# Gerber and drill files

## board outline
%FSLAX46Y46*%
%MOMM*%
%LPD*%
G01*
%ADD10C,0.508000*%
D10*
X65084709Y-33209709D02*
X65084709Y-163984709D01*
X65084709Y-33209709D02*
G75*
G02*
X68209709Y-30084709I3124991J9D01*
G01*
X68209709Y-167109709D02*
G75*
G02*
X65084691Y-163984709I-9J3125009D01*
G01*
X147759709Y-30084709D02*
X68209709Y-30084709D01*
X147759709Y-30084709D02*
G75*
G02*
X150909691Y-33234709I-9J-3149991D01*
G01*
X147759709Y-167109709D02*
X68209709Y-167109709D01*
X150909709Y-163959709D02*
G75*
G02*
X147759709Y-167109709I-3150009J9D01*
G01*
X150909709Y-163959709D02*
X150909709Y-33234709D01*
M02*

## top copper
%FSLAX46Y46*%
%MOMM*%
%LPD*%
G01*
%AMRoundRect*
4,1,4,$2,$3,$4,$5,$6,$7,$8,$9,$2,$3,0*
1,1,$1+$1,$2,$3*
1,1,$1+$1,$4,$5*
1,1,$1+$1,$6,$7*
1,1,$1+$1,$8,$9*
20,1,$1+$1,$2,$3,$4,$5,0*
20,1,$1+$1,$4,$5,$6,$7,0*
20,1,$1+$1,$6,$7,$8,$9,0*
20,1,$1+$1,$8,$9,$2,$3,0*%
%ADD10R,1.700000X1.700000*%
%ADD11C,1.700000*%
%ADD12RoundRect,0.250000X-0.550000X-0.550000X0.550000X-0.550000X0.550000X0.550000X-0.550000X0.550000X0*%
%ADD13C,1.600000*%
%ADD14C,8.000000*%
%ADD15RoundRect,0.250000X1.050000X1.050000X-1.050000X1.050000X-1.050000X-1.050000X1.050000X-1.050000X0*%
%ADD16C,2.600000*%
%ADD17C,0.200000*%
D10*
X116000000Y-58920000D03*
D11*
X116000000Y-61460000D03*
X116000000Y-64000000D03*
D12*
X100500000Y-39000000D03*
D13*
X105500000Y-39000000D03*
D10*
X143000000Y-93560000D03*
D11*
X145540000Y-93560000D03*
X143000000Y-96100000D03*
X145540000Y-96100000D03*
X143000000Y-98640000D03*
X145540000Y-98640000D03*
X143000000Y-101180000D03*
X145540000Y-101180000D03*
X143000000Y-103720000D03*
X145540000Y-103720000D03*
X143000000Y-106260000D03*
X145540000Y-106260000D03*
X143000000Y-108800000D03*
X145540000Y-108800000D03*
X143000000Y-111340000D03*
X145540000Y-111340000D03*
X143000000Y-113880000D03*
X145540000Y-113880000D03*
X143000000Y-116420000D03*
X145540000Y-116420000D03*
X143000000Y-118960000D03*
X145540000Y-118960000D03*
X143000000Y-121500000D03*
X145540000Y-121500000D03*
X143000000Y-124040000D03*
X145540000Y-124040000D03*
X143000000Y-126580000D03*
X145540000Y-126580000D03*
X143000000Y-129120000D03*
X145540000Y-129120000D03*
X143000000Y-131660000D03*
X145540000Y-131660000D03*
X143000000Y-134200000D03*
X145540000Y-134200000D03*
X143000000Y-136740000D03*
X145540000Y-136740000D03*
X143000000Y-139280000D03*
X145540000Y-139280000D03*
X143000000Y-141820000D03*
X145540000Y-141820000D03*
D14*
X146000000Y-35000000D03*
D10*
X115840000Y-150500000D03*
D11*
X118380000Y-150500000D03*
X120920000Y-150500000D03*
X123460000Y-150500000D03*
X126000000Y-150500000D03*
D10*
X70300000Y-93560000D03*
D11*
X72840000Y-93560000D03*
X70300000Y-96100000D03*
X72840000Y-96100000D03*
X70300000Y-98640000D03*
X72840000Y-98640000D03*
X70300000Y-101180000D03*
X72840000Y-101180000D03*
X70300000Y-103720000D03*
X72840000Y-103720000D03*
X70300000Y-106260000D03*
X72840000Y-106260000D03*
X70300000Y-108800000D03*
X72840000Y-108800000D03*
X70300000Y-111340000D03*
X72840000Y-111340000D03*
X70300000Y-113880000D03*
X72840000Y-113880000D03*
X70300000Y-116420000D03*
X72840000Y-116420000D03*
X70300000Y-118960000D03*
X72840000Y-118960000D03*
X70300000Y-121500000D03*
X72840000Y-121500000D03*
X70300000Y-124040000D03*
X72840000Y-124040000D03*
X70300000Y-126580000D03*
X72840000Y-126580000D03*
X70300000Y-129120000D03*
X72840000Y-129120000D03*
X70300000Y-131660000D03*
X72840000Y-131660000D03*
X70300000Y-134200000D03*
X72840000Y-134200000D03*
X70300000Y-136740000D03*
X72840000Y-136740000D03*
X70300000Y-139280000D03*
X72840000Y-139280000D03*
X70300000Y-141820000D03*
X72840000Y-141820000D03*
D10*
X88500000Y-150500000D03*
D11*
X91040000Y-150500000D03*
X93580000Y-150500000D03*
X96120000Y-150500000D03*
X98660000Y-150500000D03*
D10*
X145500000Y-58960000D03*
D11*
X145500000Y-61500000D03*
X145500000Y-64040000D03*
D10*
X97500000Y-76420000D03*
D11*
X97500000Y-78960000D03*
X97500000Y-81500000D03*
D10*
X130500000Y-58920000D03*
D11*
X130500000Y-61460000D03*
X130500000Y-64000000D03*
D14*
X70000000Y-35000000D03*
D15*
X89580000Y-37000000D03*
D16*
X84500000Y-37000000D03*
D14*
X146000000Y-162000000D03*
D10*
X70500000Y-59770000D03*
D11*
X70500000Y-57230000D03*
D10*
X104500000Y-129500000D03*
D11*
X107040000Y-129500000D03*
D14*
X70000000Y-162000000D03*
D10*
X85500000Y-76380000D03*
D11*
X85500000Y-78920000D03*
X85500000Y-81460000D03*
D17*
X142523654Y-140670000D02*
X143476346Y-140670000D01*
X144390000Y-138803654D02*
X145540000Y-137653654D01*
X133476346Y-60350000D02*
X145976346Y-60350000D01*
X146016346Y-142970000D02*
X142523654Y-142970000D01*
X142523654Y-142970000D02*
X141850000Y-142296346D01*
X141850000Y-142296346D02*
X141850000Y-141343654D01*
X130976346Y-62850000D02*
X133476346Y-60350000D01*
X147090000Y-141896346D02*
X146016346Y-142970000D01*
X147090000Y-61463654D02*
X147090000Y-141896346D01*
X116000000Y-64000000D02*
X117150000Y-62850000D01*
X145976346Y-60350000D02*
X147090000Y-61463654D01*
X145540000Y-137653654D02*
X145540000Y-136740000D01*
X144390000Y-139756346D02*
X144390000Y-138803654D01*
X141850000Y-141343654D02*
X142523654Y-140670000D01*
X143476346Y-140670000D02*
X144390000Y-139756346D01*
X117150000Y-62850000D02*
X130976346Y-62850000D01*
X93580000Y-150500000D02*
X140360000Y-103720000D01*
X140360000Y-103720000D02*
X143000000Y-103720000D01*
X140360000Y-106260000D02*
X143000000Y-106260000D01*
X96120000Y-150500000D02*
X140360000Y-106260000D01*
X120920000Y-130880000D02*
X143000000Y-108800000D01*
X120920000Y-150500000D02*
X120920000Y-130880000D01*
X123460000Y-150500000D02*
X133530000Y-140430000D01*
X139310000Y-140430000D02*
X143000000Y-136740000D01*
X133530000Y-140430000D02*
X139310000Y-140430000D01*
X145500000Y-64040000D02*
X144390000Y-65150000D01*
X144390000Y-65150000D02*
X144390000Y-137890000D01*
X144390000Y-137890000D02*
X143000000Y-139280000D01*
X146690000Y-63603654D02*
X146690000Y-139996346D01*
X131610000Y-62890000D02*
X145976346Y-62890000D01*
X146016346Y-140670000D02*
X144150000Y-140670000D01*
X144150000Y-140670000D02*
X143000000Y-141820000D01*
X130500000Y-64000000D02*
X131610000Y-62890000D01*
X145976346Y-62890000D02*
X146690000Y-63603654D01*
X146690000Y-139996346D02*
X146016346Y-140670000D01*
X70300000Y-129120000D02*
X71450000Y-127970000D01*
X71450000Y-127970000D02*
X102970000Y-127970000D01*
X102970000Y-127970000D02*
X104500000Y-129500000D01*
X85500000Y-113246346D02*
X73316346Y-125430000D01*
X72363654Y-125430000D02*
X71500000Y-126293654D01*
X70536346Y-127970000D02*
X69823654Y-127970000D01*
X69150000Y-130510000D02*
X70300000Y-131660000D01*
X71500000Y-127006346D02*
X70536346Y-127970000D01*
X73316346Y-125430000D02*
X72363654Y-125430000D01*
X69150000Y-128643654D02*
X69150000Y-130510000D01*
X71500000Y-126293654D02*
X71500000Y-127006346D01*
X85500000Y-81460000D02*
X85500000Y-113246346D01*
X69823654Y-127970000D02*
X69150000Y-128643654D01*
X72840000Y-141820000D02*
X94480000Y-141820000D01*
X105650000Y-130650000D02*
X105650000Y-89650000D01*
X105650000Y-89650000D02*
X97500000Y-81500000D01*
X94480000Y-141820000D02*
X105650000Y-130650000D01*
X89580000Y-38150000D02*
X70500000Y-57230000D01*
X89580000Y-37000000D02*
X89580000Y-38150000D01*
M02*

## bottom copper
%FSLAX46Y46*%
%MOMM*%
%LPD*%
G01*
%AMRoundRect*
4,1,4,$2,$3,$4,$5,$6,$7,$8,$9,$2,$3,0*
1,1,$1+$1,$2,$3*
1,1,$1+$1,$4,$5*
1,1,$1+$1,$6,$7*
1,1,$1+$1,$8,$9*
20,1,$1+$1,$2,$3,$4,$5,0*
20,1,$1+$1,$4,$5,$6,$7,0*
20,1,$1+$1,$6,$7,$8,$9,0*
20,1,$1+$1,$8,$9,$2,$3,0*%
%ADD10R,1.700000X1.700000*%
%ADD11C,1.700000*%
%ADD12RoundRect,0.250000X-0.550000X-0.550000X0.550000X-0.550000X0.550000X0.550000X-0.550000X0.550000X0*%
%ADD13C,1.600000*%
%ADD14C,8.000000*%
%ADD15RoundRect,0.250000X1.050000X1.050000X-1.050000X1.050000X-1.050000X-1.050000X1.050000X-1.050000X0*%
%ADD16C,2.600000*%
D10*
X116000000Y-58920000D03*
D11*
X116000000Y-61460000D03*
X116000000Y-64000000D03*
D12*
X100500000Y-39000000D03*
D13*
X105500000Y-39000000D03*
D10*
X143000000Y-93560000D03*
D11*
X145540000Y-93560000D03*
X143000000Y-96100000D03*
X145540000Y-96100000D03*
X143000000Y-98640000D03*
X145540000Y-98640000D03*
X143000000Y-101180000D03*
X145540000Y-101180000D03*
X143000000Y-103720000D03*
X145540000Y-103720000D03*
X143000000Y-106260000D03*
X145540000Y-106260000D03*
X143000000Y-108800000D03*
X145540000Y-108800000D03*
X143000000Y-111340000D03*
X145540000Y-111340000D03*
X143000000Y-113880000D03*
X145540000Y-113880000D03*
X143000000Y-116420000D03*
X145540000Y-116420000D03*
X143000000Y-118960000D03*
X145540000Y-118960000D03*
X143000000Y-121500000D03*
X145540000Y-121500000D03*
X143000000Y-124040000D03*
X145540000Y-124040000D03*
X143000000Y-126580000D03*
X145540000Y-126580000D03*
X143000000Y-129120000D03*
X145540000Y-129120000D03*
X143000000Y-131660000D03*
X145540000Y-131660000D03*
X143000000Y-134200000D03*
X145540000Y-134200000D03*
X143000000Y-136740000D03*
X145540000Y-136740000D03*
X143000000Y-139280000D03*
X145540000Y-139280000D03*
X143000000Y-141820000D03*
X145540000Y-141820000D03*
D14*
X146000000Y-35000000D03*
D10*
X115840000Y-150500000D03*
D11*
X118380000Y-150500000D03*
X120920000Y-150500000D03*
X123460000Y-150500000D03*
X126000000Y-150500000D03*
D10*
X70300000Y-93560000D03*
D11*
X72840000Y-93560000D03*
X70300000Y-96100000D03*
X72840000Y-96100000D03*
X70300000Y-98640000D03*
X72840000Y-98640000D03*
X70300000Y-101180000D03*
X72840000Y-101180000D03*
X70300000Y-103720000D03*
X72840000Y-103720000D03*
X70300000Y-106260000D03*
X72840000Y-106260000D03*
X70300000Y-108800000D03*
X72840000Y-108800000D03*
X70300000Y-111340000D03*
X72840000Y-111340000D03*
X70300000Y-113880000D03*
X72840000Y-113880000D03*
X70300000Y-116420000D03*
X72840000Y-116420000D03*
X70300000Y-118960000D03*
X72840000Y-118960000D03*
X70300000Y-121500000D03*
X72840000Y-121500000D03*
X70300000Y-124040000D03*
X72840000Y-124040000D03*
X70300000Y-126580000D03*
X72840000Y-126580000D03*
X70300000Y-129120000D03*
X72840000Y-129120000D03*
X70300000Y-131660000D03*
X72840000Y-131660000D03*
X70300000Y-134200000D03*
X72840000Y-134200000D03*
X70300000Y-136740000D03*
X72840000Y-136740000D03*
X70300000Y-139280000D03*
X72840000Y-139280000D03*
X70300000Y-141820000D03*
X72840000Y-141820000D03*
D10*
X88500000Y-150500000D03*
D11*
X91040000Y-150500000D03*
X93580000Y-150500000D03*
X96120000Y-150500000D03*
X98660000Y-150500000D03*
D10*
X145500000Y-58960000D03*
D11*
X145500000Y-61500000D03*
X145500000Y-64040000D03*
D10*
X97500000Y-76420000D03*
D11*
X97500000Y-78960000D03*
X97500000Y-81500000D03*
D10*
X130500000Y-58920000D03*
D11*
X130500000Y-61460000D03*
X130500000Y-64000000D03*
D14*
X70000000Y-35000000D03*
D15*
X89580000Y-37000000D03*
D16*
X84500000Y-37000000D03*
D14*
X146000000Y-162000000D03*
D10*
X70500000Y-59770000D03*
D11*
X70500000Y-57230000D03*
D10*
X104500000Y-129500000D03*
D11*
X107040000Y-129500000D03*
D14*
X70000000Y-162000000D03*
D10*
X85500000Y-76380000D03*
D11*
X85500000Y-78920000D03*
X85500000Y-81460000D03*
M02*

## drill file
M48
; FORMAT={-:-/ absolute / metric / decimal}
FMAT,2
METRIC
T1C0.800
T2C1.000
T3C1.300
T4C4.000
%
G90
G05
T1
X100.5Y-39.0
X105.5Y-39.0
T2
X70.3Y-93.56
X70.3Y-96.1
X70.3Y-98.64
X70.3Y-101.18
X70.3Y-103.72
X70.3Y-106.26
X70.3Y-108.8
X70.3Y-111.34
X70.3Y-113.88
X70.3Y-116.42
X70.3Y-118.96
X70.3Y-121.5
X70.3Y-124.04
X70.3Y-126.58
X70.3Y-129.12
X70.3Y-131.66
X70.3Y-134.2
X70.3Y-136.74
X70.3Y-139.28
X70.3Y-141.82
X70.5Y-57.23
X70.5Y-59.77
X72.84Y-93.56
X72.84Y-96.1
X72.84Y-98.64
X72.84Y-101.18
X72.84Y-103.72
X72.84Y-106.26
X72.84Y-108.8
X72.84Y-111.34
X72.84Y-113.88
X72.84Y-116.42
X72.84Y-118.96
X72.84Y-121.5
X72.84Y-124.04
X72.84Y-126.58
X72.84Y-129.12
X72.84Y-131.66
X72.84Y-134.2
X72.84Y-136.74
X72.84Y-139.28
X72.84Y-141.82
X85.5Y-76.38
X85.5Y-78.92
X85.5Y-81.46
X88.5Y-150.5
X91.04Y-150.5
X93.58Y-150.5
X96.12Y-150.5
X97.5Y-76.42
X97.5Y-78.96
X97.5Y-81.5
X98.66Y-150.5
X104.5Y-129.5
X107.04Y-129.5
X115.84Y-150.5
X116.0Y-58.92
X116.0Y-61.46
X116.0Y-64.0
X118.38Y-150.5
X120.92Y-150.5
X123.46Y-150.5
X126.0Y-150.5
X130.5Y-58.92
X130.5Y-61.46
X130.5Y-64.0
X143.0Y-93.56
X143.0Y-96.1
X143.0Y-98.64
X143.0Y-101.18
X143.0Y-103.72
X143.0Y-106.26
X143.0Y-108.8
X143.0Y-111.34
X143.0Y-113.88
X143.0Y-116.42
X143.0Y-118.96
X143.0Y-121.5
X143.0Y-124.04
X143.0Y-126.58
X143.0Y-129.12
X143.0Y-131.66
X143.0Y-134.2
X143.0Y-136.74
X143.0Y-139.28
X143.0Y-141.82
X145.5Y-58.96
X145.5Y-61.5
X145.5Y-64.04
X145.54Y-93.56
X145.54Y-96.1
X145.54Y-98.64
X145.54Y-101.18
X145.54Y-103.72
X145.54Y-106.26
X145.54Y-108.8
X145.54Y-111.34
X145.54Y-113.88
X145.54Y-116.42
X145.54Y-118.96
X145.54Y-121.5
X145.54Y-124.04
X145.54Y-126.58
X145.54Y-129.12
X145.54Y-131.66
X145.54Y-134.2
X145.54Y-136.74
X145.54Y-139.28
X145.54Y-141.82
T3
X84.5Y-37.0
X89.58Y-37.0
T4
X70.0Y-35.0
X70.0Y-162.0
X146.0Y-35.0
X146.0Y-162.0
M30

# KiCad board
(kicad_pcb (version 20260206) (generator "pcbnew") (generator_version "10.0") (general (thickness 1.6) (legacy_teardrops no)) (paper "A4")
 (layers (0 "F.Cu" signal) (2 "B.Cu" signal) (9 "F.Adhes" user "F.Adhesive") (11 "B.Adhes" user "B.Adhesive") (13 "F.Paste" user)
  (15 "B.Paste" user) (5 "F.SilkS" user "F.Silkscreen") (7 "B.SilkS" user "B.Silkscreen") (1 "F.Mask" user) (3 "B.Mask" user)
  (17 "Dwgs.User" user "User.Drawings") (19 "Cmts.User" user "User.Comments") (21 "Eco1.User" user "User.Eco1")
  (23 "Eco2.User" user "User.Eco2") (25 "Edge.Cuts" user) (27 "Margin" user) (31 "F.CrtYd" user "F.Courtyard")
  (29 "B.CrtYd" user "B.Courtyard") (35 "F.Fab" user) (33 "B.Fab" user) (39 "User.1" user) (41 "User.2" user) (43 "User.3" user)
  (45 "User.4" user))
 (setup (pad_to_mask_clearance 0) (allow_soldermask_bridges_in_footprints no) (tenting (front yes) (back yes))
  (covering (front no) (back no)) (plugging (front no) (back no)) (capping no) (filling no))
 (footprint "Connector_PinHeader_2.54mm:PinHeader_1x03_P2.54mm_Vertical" (layer "F.Cu") (at 116 58.92)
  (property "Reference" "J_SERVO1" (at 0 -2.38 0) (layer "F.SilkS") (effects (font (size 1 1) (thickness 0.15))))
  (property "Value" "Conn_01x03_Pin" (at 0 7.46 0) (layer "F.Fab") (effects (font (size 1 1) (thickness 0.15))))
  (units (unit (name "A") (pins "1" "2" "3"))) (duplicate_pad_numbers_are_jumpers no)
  (pad "1" thru_hole rect (at 0 0) (size 1.7 1.7) (drill 1) (layers "*.Cu" "*.Mask") (remove_unused_layers no) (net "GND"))
  (pad "2" thru_hole circle (at 0 2.54) (size 1.7 1.7) (drill 1) (layers "*.Cu" "*.Mask") (remove_unused_layers no) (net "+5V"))
  (pad "3" thru_hole circle (at 0 5.08) (size 1.7 1.7) (drill 1) (layers "*.Cu" "*.Mask") (remove_unused_layers no) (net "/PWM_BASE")))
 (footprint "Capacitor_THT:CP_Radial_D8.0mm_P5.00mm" (layer "F.Cu") (at 100.5 39)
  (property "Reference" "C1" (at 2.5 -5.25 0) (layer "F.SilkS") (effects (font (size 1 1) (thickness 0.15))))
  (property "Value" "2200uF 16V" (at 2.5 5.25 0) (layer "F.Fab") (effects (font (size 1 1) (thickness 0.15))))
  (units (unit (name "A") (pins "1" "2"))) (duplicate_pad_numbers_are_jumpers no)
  (pad "1" thru_hole roundrect (at 0 0) (size 1.6 1.6) (drill 0.8) (layers "*.Cu" "*.Mask") (remove_unused_layers no)
   (roundrect_rratio 0.15625) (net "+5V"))
  (pad "2" thru_hole circle (at 5 0) (size 1.6 1.6) (drill 0.8) (layers "*.Cu" "*.Mask") (remove_unused_layers no) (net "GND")))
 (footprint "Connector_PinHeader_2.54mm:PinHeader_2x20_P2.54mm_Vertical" (layer "F.Cu") (at 143 93.56)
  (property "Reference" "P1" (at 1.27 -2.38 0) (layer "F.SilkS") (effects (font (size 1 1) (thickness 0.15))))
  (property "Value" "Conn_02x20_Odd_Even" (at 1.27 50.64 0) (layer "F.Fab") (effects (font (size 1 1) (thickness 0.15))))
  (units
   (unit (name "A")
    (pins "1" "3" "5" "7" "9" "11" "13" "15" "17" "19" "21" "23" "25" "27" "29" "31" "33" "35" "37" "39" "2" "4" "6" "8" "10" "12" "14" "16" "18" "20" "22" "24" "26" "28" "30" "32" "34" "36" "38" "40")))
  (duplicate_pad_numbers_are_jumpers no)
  (pad "1" thru_hole rect (at 0 0) (size 1.7 1.7) (drill 1) (layers "*.Cu" "*.Mask") (remove_unused_layers no) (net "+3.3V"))
  (pad "2" thru_hole circle (at 2.54 0) (size 1.7 1.7) (drill 1) (layers "*.Cu" "*.Mask") (remove_unused_layers no) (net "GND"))
  (pad "3" thru_hole circle (at 0 2.54) (size 1.7 1.7) (drill 1) (layers "*.Cu" "*.Mask") (remove_unused_layers no)
   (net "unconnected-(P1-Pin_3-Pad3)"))
  (pad "4" thru_hole circle (at 2.54 2.54) (size 1.7 1.7) (drill 1) (layers "*.Cu" "*.Mask") (remove_unused_layers no)
   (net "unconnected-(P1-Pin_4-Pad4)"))
  (pad "5" thru_hole circle (at 0 5.08) (size 1.7 1.7) (drill 1) (layers "*.Cu" "*.Mask") (remove_unused_layers no)
   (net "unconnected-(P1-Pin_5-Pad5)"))
  (pad "6" thru_hole circle (at 2.54 5.08) (size 1.7 1.7) (drill 1) (layers "*.Cu" "*.Mask") (remove_unused_layers no)
   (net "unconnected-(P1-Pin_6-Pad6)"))
  (pad "7" thru_hole circle (at 0 7.62) (size 1.7 1.7) (drill 1) (layers "*.Cu" "*.Mask") (remove_unused_layers no) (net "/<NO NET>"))
  (pad "8" thru_hole circle (at 2.54 7.62) (size 1.7 1.7) (drill 1) (layers "*.Cu" "*.Mask") (remove_unused_layers no)
   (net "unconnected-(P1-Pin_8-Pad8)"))
  (pad "9" thru_hole circle (at 0 10.16) (size 1.7 1.7) (drill 1) (layers "*.Cu" "*.Mask") (remove_unused_layers no) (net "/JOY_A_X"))
  (pad "10" thru_hole circle (at 2.54 10.16) (size 1.7 1.7) (drill 1) (layers "*.Cu" "*.Mask") (remove_unused_layers no)
   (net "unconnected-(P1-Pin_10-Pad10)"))
  (pad "11" thru_hole circle (at 0 12.7) (size 1.7 1.7) (drill 1) (layers "*.Cu" "*.Mask") (remove_unused_layers no) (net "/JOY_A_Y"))
  (pad "12" thru_hole circle (at 2.54 12.7) (size 1.7 1.7) (drill 1) (layers "*.Cu" "*.Mask") (remove_unused_layers no)
   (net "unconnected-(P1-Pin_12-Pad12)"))
  (pad "13" thru_hole circle (at 0 15.24) (size 1.7 1.7) (drill 1) (layers "*.Cu" "*.Mask") (remove_unused_layers no) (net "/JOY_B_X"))
  (pad "14" thru_hole circle (at 2.54 15.24) (size 1.7 1.7) (drill 1) (layers "*.Cu" "*.Mask") (remove_unused_layers no)
   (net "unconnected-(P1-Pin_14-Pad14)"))
  (pad "15" thru_hole circle (at 0 17.78) (size 1.7 1.7) (drill 1) (layers "*.Cu" "*.Mask") (remove_unused_layers no)
   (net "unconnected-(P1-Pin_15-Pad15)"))
  (pad "16" thru_hole circle (at 2.54 17.78) (size 1.7 1.7) (drill 1) (layers "*.Cu" "*.Mask") (remove_unused_layers no)
   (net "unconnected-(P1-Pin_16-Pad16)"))
  (pad "17" thru_hole circle (at 0 20.32) (size 1.7 1.7) (drill 1) (layers "*.Cu" "*.Mask") (remove_unused_layers no)
   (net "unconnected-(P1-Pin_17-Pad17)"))
  (pad "18" thru_hole circle (at 2.54 20.32) (size 1.7 1.7) (drill 1) (layers "*.Cu" "*.Mask") (remove_unused_layers no)
   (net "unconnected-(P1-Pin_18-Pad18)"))
  (pad "19" thru_hole circle (at 0 22.86) (size 1.7 1.7) (drill 1) (layers "*.Cu" "*.Mask") (remove_unused_layers no)
   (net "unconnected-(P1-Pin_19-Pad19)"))
  (pad "20" thru_hole circle (at 2.54 22.86) (size 1.7 1.7) (drill 1) (layers "*.Cu" "*.Mask") (remove_unused_layers no)
   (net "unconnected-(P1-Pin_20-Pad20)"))
  (pad "21" thru_hole circle (at 0 25.4) (size 1.7 1.7) (drill 1) (layers "*.Cu" "*.Mask") (remove_unused_layers no)
   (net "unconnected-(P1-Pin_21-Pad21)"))
  (pad "22" thru_hole circle (at 2.54 25.4) (size 1.7 1.7) (drill 1) (layers "*.Cu" "*.Mask") (remove_unused_layers no)
   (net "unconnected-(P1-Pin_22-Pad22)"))
  (pad "23" thru_hole circle (at 0 27.94) (size 1.7 1.7) (drill 1) (layers "*.Cu" "*.Mask") (remove_unused_layers no)
   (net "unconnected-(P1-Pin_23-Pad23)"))
  (pad "24" thru_hole circle (at 2.54 27.94) (size 1.7 1.7) (drill 1) (layers "*.Cu" "*.Mask") (remove_unused_layers no)
   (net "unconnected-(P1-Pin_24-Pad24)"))
  (pad "25" thru_hole circle (at 0 30.48) (size 1.7 1.7) (drill 1) (layers "*.Cu" "*.Mask") (remove_unused_layers no)
   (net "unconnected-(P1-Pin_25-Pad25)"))
  (pad "26" thru_hole circle (at 2.54 30.48) (size 1.7 1.7) (drill 1) (layers "*.Cu" "*.Mask") (remove_unused_layers no)
   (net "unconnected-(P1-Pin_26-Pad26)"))
  (pad "27" thru_hole circle (at 0 33.02) (size 1.7 1.7) (drill 1) (layers "*.Cu" "*.Mask") (remove_unused_layers no)
   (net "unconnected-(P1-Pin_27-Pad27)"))
  (pad "28" thru_hole circle (at 2.54 33.02) (size 1.7 1.7) (drill 1) (layers "*.Cu" "*.Mask") (remove_unused_layers no)
   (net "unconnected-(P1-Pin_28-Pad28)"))
  (pad "29" thru_hole circle (at 0 35.56) (size 1.7 1.7) (drill 1) (layers "*.Cu" "*.Mask") (remove_unused_layers no)
   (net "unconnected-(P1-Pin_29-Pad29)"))
  (pad "30" thru_hole circle (at 2.54 35.56) (size 1.7 1.7) (drill 1) (layers "*.Cu" "*.Mask") (remove_unused_layers no)
   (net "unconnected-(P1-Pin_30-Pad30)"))
  (pad "31" thru_hole circle (at 0 38.1) (size 1.7 1.7) (drill 1) (layers "*.Cu" "*.Mask") (remove_unused_layers no)
   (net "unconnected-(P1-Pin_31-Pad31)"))
  (pad "32" thru_hole circle (at 2.54 38.1) (size 1.7 1.7) (drill 1) (layers "*.Cu" "*.Mask") (remove_unused_layers no)
   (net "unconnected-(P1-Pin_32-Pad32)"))
  (pad "33" thru_hole circle (at 0 40.64) (size 1.7 1.7) (drill 1) (layers "*.Cu" "*.Mask") (remove_unused_layers no)
   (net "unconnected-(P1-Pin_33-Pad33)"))
  (pad "34" thru_hole circle (at 2.54 40.64) (size 1.7 1.7) (drill 1) (layers "*.Cu" "*.Mask") (remove_unused_layers no)
   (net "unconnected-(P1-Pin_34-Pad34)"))
  (pad "35" thru_hole circle (at 0 43.18) (size 1.7 1.7) (drill 1) (layers "*.Cu" "*.Mask") (remove_unused_layers no) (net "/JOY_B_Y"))
  (pad "36" thru_hole circle (at 2.54 43.18) (size 1.7 1.7) (drill 1) (layers "*.Cu" "*.Mask") (remove_unused_layers no) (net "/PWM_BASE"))
  (pad "37" thru_hole circle (at 0 45.72) (size 1.7 1.7) (drill 1) (layers "*.Cu" "*.Mask") (remove_unused_layers no) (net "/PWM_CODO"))
  (pad "38" thru_hole circle (at 2.54 45.72) (size 1.7 1.7) (drill 1) (layers "*.Cu" "*.Mask") (remove_unused_layers no)
   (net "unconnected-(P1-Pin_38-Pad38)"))
  (pad "39" thru_hole circle (at 0 48.26) (size 1.7 1.7) (drill 1) (layers "*.Cu" "*.Mask") (remove_unused_layers no) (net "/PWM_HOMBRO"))
  (pad "40" thru_hole circle (at 2.54 48.26) (size 1.7 1.7) (drill 1) (layers "*.Cu" "*.Mask") (remove_unused_layers no)
   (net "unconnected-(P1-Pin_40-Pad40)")))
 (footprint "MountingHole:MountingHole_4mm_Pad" (layer "F.Cu") (at 146 35)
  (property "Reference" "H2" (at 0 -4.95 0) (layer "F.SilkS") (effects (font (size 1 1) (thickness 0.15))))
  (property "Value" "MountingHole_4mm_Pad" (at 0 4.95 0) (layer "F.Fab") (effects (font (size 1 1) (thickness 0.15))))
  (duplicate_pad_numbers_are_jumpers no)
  (pad "1" thru_hole circle (at 0 0) (size 8 8) (drill 4) (layers "*.Cu" "*.Mask") (remove_unused_layers no) (zone_connect 2)))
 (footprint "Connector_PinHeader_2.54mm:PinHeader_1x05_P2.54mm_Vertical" (layer "F.Cu") (at 115.84 150.5 90)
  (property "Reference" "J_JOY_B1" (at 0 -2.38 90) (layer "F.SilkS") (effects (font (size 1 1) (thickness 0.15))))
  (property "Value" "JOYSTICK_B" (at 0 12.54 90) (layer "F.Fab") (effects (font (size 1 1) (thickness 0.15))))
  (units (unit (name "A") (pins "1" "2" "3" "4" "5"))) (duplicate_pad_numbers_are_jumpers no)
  (pad "1" thru_hole rect (at 0 0 90) (size 1.7 1.7) (drill 1) (layers "*.Cu" "*.Mask") (remove_unused_layers no) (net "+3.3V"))
  (pad "2" thru_hole circle (at 0 2.54 90) (size 1.7 1.7) (drill 1) (layers "*.Cu" "*.Mask") (remove_unused_layers no) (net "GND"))
  (pad "3" thru_hole circle (at 0 5.08 90) (size 1.7 1.7) (drill 1) (layers "*.Cu" "*.Mask") (remove_unused_layers no) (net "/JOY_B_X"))
  (pad "4" thru_hole circle (at 0 7.62 90) (size 1.7 1.7) (drill 1) (layers "*.Cu" "*.Mask") (remove_unused_layers no) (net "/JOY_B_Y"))
  (pad "5" thru_hole circle (at 0 10.16 90) (size 1.7 1.7) (drill 1) (layers "*.Cu" "*.Mask") (remove_unused_layers no)
   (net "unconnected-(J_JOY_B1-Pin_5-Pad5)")))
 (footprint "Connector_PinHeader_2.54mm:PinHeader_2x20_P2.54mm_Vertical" (layer "F.Cu") (at 70.3 93.56)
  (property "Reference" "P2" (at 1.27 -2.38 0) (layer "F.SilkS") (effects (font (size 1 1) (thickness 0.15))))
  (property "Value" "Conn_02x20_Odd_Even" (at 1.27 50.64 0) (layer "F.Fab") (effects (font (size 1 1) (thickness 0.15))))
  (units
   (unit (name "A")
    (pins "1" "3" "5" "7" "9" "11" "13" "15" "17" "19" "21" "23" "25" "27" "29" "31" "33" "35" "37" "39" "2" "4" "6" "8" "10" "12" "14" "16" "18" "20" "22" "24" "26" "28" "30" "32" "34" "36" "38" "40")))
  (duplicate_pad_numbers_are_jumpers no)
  (pad "1" thru_hole rect (at 0 0) (size 1.7 1.7) (drill 1) (layers "*.Cu" "*.Mask") (remove_unused_layers no)
   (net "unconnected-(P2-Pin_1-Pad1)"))
  (pad "2" thru_hole circle (at 2.54 0) (size 1.7 1.7) (drill 1) (layers "*.Cu" "*.Mask") (remove_unused_layers no)
   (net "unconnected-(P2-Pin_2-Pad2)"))
  (pad "3" thru_hole circle (at 0 2.54) (size 1.7 1.7) (drill 1) (layers "*.Cu" "*.Mask") (remove_unused_layers no)
   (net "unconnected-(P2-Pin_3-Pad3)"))
  (pad "4" thru_hole circle (at 2.54 2.54) (size 1.7 1.7) (drill 1) (layers "*.Cu" "*.Mask") (remove_unused_layers no)
   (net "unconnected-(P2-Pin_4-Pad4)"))
  (pad "5" thru_hole circle (at 0 5.08) (size 1.7 1.7) (drill 1) (layers "*.Cu" "*.Mask") (remove_unused_layers no)
   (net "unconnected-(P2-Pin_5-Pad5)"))
  (pad "6" thru_hole circle (at 2.54 5.08) (size 1.7 1.7) (drill 1) (layers "*.Cu" "*.Mask") (remove_unused_layers no)
   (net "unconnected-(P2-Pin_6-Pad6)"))
  (pad "7" thru_hole circle (at 0 7.62) (size 1.7 1.7) (drill 1) (layers "*.Cu" "*.Mask") (remove_unused_layers no)
   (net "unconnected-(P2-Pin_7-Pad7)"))
  (pad "8" thru_hole circle (at 2.54 7.62) (size 1.7 1.7) (drill 1) (layers "*.Cu" "*.Mask") (remove_unused_layers no)
   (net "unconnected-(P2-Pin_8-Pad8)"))
  (pad "9" thru_hole circle (at 0 10.16) (size 1.7 1.7) (drill 1) (layers "*.Cu" "*.Mask") (remove_unused_layers no)
   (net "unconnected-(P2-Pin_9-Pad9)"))
  (pad "10" thru_hole circle (at 2.54 10.16) (size 1.7 1.7) (drill 1) (layers "*.Cu" "*.Mask") (remove_unused_layers no)
   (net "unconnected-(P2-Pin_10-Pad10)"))
  (pad "11" thru_hole circle (at 0 12.7) (size 1.7 1.7) (drill 1) (layers "*.Cu" "*.Mask") (remove_unused_layers no)
   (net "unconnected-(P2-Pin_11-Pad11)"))
  (pad "12" thru_hole circle (at 2.54 12.7) (size 1.7 1.7) (drill 1) (layers "*.Cu" "*.Mask") (remove_unused_layers no)
   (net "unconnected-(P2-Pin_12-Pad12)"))
  (pad "13" thru_hole circle (at 0 15.24) (size 1.7 1.7) (drill 1) (layers "*.Cu" "*.Mask") (remove_unused_layers no)
   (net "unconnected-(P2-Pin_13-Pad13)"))
  (pad "14" thru_hole circle (at 2.54 15.24) (size 1.7 1.7) (drill 1) (layers "*.Cu" "*.Mask") (remove_unused_layers no)
   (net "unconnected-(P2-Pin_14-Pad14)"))
  (pad "15" thru_hole circle (at 0 17.78) (size 1.7 1.7) (drill 1) (layers "*.Cu" "*.Mask") (remove_unused_layers no)
   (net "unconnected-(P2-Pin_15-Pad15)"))
  (pad "16" thru_hole circle (at 2.54 17.78) (size 1.7 1.7) (drill 1) (layers "*.Cu" "*.Mask") (remove_unused_layers no)
   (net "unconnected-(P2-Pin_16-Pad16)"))
  (pad "17" thru_hole circle (at 0 20.32) (size 1.7 1.7) (drill 1) (layers "*.Cu" "*.Mask") (remove_unused_layers no)
   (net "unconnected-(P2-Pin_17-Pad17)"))
  (pad "18" thru_hole circle (at 2.54 20.32) (size 1.7 1.7) (drill 1) (layers "*.Cu" "*.Mask") (remove_unused_layers no)
   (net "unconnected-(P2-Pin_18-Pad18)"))
  (pad "19" thru_hole circle (at 0 22.86) (size 1.7 1.7) (drill 1) (layers "*.Cu" "*.Mask") (remove_unused_layers no)
   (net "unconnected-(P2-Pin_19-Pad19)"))
  (pad "20" thru_hole circle (at 2.54 22.86) (size 1.7 1.7) (drill 1) (layers "*.Cu" "*.Mask") (remove_unused_layers no)
   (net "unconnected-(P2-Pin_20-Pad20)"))
  (pad "21" thru_hole circle (at 0 25.4) (size 1.7 1.7) (drill 1) (layers "*.Cu" "*.Mask") (remove_unused_layers no)
   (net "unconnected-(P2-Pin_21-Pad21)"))
  (pad "22" thru_hole circle (at 2.54 25.4) (size 1.7 1.7) (drill 1) (layers "*.Cu" "*.Mask") (remove_unused_layers no)
   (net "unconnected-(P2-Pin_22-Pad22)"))
  (pad "23" thru_hole circle (at 0 27.94) (size 1.7 1.7) (drill 1) (layers "*.Cu" "*.Mask") (remove_unused_layers no)
   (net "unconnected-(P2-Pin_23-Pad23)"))
  (pad "24" thru_hole circle (at 2.54 27.94) (size 1.7 1.7) (drill 1) (layers "*.Cu" "*.Mask") (remove_unused_layers no)
   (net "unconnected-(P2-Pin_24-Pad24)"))
  (pad "25" thru_hole circle (at 0 30.48) (size 1.7 1.7) (drill 1) (layers "*.Cu" "*.Mask") (remove_unused_layers no)
   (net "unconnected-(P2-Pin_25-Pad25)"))
  (pad "26" thru_hole circle (at 2.54 30.48) (size 1.7 1.7) (drill 1) (layers "*.Cu" "*.Mask") (remove_unused_layers no)
   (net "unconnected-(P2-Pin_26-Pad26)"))
  (pad "27" thru_hole circle (at 0 33.02) (size 1.7 1.7) (drill 1) (layers "*.Cu" "*.Mask") (remove_unused_layers no) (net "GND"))
  (pad "28" thru_hole circle (at 2.54 33.02) (size 1.7 1.7) (drill 1) (layers "*.Cu" "*.Mask") (remove_unused_layers no)
   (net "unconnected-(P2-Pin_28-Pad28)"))
  (pad "29" thru_hole circle (at 0 35.56) (size 1.7 1.7) (drill 1) (layers "*.Cu" "*.Mask") (remove_unused_layers no) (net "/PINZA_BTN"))
  (pad "30" thru_hole circle (at 2.54 35.56) (size 1.7 1.7) (drill 1) (layers "*.Cu" "*.Mask") (remove_unused_layers no)
   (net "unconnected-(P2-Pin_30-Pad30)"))
  (pad "31" thru_hole circle (at 0 38.1) (size 1.7 1.7) (drill 1) (layers "*.Cu" "*.Mask") (remove_unused_layers no) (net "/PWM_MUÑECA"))
  (pad "32" thru_hole circle (at 2.54 38.1) (size 1.7 1.7) (drill 1) (layers "*.Cu" "*.Mask") (remove_unused_layers no)
   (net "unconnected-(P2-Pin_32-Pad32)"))
  (pad "33" thru_hole circle (at 0 40.64) (size 1.7 1.7) (drill 1) (layers "*.Cu" "*.Mask") (remove_unused_layers no)
   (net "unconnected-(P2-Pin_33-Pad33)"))
  (pad "34" thru_hole circle (at 2.54 40.64) (size 1.7 1.7) (drill 1) (layers "*.Cu" "*.Mask") (remove_unused_layers no)
   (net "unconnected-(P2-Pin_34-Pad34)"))
  (pad "35" thru_hole circle (at 0 43.18) (size 1.7 1.7) (drill 1) (layers "*.Cu" "*.Mask") (remove_unused_layers no)
   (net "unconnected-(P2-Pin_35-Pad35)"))
  (pad "36" thru_hole circle (at 2.54 43.18) (size 1.7 1.7) (drill 1) (layers "*.Cu" "*.Mask") (remove_unused_layers no)
   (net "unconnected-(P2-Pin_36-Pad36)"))
  (pad "37" thru_hole circle (at 0 45.72) (size 1.7 1.7) (drill 1) (layers "*.Cu" "*.Mask") (remove_unused_layers no)
   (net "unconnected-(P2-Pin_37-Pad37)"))
  (pad "38" thru_hole circle (at 2.54 45.72) (size 1.7 1.7) (drill 1) (layers "*.Cu" "*.Mask") (remove_unused_layers no)
   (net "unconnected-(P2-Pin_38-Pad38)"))
  (pad "39" thru_hole circle (at 0 48.26) (size 1.7 1.7) (drill 1) (layers "*.Cu" "*.Mask") (remove_unused_layers no)
   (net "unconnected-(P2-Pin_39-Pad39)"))
  (pad "40" thru_hole circle (at 2.54 48.26) (size 1.7 1.7) (drill 1) (layers "*.Cu" "*.Mask") (remove_unused_layers no) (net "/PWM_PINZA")))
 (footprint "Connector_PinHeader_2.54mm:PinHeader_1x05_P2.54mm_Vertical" (layer "F.Cu") (at 88.5 150.5 90)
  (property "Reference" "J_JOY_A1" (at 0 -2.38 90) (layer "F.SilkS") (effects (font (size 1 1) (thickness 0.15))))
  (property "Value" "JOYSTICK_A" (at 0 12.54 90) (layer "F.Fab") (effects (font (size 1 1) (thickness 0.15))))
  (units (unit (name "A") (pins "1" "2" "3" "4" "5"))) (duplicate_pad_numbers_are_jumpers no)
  (pad "1" thru_hole rect (at 0 0 90) (size 1.7 1.7) (drill 1) (layers "*.Cu" "*.Mask") (remove_unused_layers no) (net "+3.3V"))
  (pad "2" thru_hole circle (at 0 2.54 90) (size 1.7 1.7) (drill 1) (layers "*.Cu" "*.Mask") (remove_unused_layers no) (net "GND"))
  (pad "3" thru_hole circle (at 0 5.08 90) (size 1.7 1.7) (drill 1) (layers "*.Cu" "*.Mask") (remove_unused_layers no) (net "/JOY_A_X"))
  (pad "4" thru_hole circle (at 0 7.62 90) (size 1.7 1.7) (drill 1) (layers "*.Cu" "*.Mask") (remove_unused_layers no) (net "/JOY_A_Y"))
  (pad "5" thru_hole circle (at 0 10.16 90) (size 1.7 1.7) (drill 1) (layers "*.Cu" "*.Mask") (remove_unused_layers no)
   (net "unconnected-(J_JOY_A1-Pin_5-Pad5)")))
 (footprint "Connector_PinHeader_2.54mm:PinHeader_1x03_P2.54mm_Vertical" (layer "F.Cu") (at 145.5 58.96)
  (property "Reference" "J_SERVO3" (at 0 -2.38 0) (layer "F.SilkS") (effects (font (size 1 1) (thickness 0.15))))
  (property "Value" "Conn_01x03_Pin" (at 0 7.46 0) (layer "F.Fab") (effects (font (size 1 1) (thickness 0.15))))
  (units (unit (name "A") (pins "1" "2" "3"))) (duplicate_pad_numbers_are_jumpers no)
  (pad "1" thru_hole rect (at 0 0) (size 1.7 1.7) (drill 1) (layers "*.Cu" "*.Mask") (remove_unused_layers no) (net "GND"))
  (pad "2" thru_hole circle (at 0 2.54) (size 1.7 1.7) (drill 1) (layers "*.Cu" "*.Mask") (remove_unused_layers no) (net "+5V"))
  (pad "3" thru_hole circle (at 0 5.08) (size 1.7 1.7) (drill 1) (layers "*.Cu" "*.Mask") (remove_unused_layers no) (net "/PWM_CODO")))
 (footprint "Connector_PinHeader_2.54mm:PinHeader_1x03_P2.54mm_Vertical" (layer "F.Cu") (at 97.5 76.42)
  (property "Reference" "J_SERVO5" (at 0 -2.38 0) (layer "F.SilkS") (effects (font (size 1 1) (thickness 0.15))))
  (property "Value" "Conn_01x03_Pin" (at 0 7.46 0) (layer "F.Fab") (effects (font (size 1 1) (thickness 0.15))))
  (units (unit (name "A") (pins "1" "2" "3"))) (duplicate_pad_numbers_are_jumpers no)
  (pad "1" thru_hole rect (at 0 0) (size 1.7 1.7) (drill 1) (layers "*.Cu" "*.Mask") (remove_unused_layers no) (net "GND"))
  (pad "2" thru_hole circle (at 0 2.54) (size 1.7 1.7) (drill 1) (layers "*.Cu" "*.Mask") (remove_unused_layers no) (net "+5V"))
  (pad "3" thru_hole circle (at 0 5.08) (size 1.7 1.7) (drill 1) (layers "*.Cu" "*.Mask") (remove_unused_layers no) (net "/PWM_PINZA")))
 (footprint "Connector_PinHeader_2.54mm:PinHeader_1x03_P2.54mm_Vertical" (layer "F.Cu") (at 130.5 58.92)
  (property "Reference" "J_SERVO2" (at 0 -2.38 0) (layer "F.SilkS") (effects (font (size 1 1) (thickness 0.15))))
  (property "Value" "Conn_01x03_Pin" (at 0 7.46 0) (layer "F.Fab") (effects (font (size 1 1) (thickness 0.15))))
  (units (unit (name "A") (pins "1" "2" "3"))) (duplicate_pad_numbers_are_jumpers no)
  (pad "1" thru_hole rect (at 0 0) (size 1.7 1.7) (drill 1) (layers "*.Cu" "*.Mask") (remove_unused_layers no) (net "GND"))
  (pad "2" thru_hole circle (at 0 2.54) (size 1.7 1.7) (drill 1) (layers "*.Cu" "*.Mask") (remove_unused_layers no) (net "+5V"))
  (pad "3" thru_hole circle (at 0 5.08) (size 1.7 1.7) (drill 1) (layers "*.Cu" "*.Mask") (remove_unused_layers no) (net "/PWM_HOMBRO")))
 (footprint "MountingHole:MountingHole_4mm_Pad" (layer "F.Cu") (at 70 35)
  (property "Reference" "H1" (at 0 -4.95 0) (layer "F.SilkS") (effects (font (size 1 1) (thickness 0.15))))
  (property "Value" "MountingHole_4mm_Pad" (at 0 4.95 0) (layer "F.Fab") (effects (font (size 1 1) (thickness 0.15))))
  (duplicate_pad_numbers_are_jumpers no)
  (pad "1" thru_hole circle (at 0 0) (size 8 8) (drill 4) (layers "*.Cu" "*.Mask") (remove_unused_layers no) (zone_connect 2)))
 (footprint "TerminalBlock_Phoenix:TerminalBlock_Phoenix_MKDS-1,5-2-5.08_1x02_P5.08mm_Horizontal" (layer "F.Cu") (at 89.58 37 180)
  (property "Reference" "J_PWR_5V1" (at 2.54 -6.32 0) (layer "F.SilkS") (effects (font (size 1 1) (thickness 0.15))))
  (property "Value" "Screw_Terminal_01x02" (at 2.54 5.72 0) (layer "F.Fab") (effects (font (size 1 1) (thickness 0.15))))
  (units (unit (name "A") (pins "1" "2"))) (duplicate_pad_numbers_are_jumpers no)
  (pad "1" thru_hole roundrect (at 0 0 180) (size 2.6 2.6) (drill 1.3) (layers "*.Cu" "*.Mask") (remove_unused_layers no)
   (roundrect_rratio 0.096154) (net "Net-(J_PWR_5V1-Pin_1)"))
  (pad "2" thru_hole circle (at 5.08 0 180) (size 2.6 2.6) (drill 1.3) (layers "*.Cu" "*.Mask") (remove_unused_layers no) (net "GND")))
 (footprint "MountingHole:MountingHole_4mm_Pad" (layer "F.Cu") (at 146 162)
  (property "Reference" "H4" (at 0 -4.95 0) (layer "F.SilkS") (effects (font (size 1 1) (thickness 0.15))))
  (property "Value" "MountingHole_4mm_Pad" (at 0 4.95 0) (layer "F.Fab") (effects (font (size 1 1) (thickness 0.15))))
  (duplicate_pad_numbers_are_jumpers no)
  (pad "1" thru_hole circle (at 0 0) (size 8 8) (drill 4) (layers "*.Cu" "*.Mask") (remove_unused_layers no) (zone_connect 2)))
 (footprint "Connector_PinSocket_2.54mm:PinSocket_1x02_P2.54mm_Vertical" (layer "F.Cu") (at 70.5 59.77 180)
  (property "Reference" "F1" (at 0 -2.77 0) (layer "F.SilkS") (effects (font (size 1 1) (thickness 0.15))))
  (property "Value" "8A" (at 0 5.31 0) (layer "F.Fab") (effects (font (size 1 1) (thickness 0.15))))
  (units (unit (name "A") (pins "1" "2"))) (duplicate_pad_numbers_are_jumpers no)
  (pad "1" thru_hole rect (at 0 0 180) (size 1.7 1.7) (drill 1) (layers "*.Cu" "*.Mask") (remove_unused_layers no) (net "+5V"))
  (pad "2" thru_hole circle (at 0 2.54 180) (size 1.7 1.7) (drill 1) (layers "*.Cu" "*.Mask") (remove_unused_layers no)
   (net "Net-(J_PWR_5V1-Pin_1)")))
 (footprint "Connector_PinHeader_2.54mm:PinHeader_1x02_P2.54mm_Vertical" (layer "F.Cu") (at 104.5 129.5 90)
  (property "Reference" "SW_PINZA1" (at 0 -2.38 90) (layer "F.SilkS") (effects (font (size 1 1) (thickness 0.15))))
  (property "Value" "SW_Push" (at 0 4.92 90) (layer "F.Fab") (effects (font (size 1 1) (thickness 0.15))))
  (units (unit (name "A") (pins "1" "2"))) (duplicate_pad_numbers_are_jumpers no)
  (pad "1" thru_hole rect (at 0 0 90) (size 1.7 1.7) (drill 1) (layers "*.Cu" "*.Mask") (remove_unused_layers no) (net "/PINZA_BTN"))
  (pad "2" thru_hole circle (at 0 2.54 90) (size 1.7 1.7) (drill 1) (layers "*.Cu" "*.Mask") (remove_unused_layers no) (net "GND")))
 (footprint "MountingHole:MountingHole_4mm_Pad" (layer "F.Cu") (at 70 162)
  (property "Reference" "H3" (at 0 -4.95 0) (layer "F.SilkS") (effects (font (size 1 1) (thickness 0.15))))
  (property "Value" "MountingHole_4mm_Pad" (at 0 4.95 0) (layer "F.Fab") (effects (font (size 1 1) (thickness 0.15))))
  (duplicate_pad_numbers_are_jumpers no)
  (pad "1" thru_hole circle (at 0 0) (size 8 8) (drill 4) (layers "*.Cu" "*.Mask") (remove_unused_layers no) (zone_connect 2)))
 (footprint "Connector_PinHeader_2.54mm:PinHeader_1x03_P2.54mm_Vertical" (layer "F.Cu") (at 85.5 76.38)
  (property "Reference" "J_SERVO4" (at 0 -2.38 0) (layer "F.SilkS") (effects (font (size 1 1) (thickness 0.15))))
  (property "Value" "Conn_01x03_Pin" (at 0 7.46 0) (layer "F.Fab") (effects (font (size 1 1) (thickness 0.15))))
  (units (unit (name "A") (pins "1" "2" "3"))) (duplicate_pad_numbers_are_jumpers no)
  (pad "1" thru_hole rect (at 0 0) (size 1.7 1.7) (drill 1) (layers "*.Cu" "*.Mask") (remove_unused_layers no) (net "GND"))
  (pad "2" thru_hole circle (at 0 2.54) (size 1.7 1.7) (drill 1) (layers "*.Cu" "*.Mask") (remove_unused_layers no) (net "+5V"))
  (pad "3" thru_hole circle (at 0 5.08) (size 1.7 1.7) (drill 1) (layers "*.Cu" "*.Mask") (remove_unused_layers no) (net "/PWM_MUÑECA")))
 (gr_line (start 65.084709 33.209709) (end 65.084709 163.984709) (stroke (width 0.508) (type solid)) (layer "Edge.Cuts"))
 (gr_arc (start 65.084709 33.209709) (mid 65.999998 30.999998) (end 68.209709 30.084709) (stroke (width 0.508) (type solid))
  (layer "Edge.Cuts"))
 (gr_arc (start 68.209709 167.109709) (mid 66 166.194418) (end 65.084709 163.984709) (stroke (width 0.508) (type solid)) (layer "Edge.Cuts"))
 (gr_line (start 147.759709 30.084709) (end 68.209709 30.084709) (stroke (width 0.508) (type solid)) (layer "Edge.Cuts"))
 (gr_arc (start 147.759709 30.084709) (mid 149.987095 31.007323) (end 150.909709 33.234709) (stroke (width 0.508) (type solid))
  (layer "Edge.Cuts"))
 (gr_line (start 147.759709 167.109709) (end 68.209709 167.109709) (stroke (width 0.508) (type solid)) (layer "Edge.Cuts"))
 (gr_arc (start 150.909709 163.959709) (mid 149.987095 166.187095) (end 147.759709 167.109709) (stroke (width 0.508) (type solid))
  (layer "Edge.Cuts"))
 (gr_line (start 150.909709 163.959709) (end 150.909709 33.234709) (stroke (width 0.508) (type solid)) (layer "Edge.Cuts"))
 (segment (start 142.523654 140.67) (end 143.476346 140.67) (width 0.2) (layer "F.Cu") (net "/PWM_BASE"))
 (segment (start 144.39 138.803654) (end 145.54 137.653654) (width 0.2) (layer "F.Cu") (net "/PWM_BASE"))
 (segment (start 133.476346 60.35) (end 145.976346 60.35) (width 0.2) (layer "F.Cu") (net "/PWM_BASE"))
 (segment (start 146.016346 142.97) (end 142.523654 142.97) (width 0.2) (layer "F.Cu") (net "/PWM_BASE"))
 (segment (start 142.523654 142.97) (end 141.85 142.296346) (width 0.2) (layer "F.Cu") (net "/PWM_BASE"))
 (segment (start 141.85 142.296346) (end 141.85 141.343654) (width 0.2) (layer "F.Cu") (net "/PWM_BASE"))
 (segment (start 130.976346 62.85) (end 133.476346 60.35) (width 0.2) (layer "F.Cu") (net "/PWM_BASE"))
 (segment (start 147.09 141.896346) (end 146.016346 142.97) (width 0.2) (layer "F.Cu") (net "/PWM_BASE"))
 (segment (start 147.09 61.463654) (end 147.09 141.896346) (width 0.2) (layer "F.Cu") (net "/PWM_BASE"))
 (segment (start 116 64) (end 117.15 62.85) (width 0.2) (layer "F.Cu") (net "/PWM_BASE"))
 (segment (start 145.976346 60.35) (end 147.09 61.463654) (width 0.2) (layer "F.Cu") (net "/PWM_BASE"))
 (segment (start 145.54 137.653654) (end 145.54 136.74) (width 0.2) (layer "F.Cu") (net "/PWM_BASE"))
 (segment (start 144.39 139.756346) (end 144.39 138.803654) (width 0.2) (layer "F.Cu") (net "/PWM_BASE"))
 (segment (start 141.85 141.343654) (end 142.523654 140.67) (width 0.2) (layer "F.Cu") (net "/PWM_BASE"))
 (segment (start 143.476346 140.67) (end 144.39 139.756346) (width 0.2) (layer "F.Cu") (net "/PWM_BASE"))
 (segment (start 117.15 62.85) (end 130.976346 62.85) (width 0.2) (layer "F.Cu") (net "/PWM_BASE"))
 (segment (start 93.58 150.5) (end 140.36 103.72) (width 0.2) (layer "F.Cu") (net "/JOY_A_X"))
 (segment (start 140.36 103.72) (end 143 103.72) (width 0.2) (layer "F.Cu") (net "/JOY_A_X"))
 (segment (start 140.36 106.26) (end 143 106.26) (width 0.2) (layer "F.Cu") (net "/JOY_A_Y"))
 (segment (start 96.12 150.5) (end 140.36 106.26) (width 0.2) (layer "F.Cu") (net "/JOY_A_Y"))
 (segment (start 120.92 130.88) (end 143 108.8) (width 0.2) (layer "F.Cu") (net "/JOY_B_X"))
 (segment (start 120.92 150.5) (end 120.92 130.88) (width 0.2) (layer "F.Cu") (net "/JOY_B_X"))
 (segment (start 123.46 150.5) (end 133.53 140.43) (width 0.2) (layer "F.Cu") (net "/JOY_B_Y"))
 (segment (start 139.31 140.43) (end 143 136.74) (width 0.2) (layer "F.Cu") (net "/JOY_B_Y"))
 (segment (start 133.53 140.43) (end 139.31 140.43) (width 0.2) (layer "F.Cu") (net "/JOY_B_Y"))
 (segment (start 145.5 64.04) (end 144.39 65.15) (width 0.2) (layer "F.Cu") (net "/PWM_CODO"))
 (segment (start 144.39 65.15) (end 144.39 137.89) (width 0.2) (layer "F.Cu") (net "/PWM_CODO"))
 (segment (start 144.39 137.89) (end 143 139.28) (width 0.2) (layer "F.Cu") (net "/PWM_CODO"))
 (segment (start 146.69 63.603654) (end 146.69 139.996346) (width 0.2) (layer "F.Cu") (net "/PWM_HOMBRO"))
 (segment (start 131.61 62.89) (end 145.976346 62.89) (width 0.2) (layer "F.Cu") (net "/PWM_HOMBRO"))
 (segment (start 146.016346 140.67) (end 144.15 140.67) (width 0.2) (layer "F.Cu") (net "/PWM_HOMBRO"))
 (segment (start 144.15 140.67) (end 143 141.82) (width 0.2) (layer "F.Cu") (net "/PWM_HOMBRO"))
 (segment (start 130.5 64) (end 131.61 62.89) (width 0.2) (layer "F.Cu") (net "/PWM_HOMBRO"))
 (segment (start 145.976346 62.89) (end 146.69 63.603654) (width 0.2) (layer "F.Cu") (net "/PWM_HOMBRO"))
 (segment (start 146.69 139.996346) (end 146.016346 140.67) (width 0.2) (layer "F.Cu") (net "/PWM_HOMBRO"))
 (segment (start 70.3 129.12) (end 71.45 127.97) (width 0.2) (layer "F.Cu") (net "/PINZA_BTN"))
 (segment (start 71.45 127.97) (end 102.97 127.97) (width 0.2) (layer "F.Cu") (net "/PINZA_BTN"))
 (segment (start 102.97 127.97) (end 104.5 129.5) (width 0.2) (layer "F.Cu") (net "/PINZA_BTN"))
 (segment (start 85.5 113.246346) (end 73.316346 125.43) (width 0.2) (layer "F.Cu") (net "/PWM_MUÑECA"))
 (segment (start 72.363654 125.43) (end 71.5 126.293654) (width 0.2) (layer "F.Cu") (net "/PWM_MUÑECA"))
 (segment (start 70.536346 127.97) (end 69.823654 127.97) (width 0.2) (layer "F.Cu") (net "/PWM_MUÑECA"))
 (segment (start 69.15 130.51) (end 70.3 131.66) (width 0.2) (layer "F.Cu") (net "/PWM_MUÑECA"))
 (segment (start 71.5 127.006346) (end 70.536346 127.97) (width 0.2) (layer "F.Cu") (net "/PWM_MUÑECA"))
 (segment (start 73.316346 125.43) (end 72.363654 125.43) (width 0.2) (layer "F.Cu") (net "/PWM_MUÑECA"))
 (segment (start 69.15 128.643654) (end 69.15 130.51) (width 0.2) (layer "F.Cu") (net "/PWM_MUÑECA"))
 (segment (start 71.5 126.293654) (end 71.5 127.006346) (width 0.2) (layer "F.Cu") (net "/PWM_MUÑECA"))
 (segment (start 85.5 81.46) (end 85.5 113.246346) (width 0.2) (layer "F.Cu") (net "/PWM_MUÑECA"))
 (segment (start 69.823654 127.97) (end 69.15 128.643654) (width 0.2) (layer "F.Cu") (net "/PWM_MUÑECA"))
 (segment (start 72.84 141.82) (end 94.48 141.82) (width 0.2) (layer "F.Cu") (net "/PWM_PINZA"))
 (segment (start 105.65 130.65) (end 105.65 89.65) (width 0.2) (layer "F.Cu") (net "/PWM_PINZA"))
 (segment (start 105.65 89.65) (end 97.5 81.5) (width 0.2) (layer "F.Cu") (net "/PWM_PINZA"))
 (segment (start 94.48 141.82) (end 105.65 130.65) (width 0.2) (layer "F.Cu") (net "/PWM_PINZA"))
 (segment (start 89.58 38.15) (end 70.5 57.23) (width 0.2) (layer "F.Cu") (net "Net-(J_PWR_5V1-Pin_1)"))
 (segment (start 89.58 37) (end 89.58 38.15) (width 0.2) (layer "F.Cu") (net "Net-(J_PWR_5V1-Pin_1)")))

